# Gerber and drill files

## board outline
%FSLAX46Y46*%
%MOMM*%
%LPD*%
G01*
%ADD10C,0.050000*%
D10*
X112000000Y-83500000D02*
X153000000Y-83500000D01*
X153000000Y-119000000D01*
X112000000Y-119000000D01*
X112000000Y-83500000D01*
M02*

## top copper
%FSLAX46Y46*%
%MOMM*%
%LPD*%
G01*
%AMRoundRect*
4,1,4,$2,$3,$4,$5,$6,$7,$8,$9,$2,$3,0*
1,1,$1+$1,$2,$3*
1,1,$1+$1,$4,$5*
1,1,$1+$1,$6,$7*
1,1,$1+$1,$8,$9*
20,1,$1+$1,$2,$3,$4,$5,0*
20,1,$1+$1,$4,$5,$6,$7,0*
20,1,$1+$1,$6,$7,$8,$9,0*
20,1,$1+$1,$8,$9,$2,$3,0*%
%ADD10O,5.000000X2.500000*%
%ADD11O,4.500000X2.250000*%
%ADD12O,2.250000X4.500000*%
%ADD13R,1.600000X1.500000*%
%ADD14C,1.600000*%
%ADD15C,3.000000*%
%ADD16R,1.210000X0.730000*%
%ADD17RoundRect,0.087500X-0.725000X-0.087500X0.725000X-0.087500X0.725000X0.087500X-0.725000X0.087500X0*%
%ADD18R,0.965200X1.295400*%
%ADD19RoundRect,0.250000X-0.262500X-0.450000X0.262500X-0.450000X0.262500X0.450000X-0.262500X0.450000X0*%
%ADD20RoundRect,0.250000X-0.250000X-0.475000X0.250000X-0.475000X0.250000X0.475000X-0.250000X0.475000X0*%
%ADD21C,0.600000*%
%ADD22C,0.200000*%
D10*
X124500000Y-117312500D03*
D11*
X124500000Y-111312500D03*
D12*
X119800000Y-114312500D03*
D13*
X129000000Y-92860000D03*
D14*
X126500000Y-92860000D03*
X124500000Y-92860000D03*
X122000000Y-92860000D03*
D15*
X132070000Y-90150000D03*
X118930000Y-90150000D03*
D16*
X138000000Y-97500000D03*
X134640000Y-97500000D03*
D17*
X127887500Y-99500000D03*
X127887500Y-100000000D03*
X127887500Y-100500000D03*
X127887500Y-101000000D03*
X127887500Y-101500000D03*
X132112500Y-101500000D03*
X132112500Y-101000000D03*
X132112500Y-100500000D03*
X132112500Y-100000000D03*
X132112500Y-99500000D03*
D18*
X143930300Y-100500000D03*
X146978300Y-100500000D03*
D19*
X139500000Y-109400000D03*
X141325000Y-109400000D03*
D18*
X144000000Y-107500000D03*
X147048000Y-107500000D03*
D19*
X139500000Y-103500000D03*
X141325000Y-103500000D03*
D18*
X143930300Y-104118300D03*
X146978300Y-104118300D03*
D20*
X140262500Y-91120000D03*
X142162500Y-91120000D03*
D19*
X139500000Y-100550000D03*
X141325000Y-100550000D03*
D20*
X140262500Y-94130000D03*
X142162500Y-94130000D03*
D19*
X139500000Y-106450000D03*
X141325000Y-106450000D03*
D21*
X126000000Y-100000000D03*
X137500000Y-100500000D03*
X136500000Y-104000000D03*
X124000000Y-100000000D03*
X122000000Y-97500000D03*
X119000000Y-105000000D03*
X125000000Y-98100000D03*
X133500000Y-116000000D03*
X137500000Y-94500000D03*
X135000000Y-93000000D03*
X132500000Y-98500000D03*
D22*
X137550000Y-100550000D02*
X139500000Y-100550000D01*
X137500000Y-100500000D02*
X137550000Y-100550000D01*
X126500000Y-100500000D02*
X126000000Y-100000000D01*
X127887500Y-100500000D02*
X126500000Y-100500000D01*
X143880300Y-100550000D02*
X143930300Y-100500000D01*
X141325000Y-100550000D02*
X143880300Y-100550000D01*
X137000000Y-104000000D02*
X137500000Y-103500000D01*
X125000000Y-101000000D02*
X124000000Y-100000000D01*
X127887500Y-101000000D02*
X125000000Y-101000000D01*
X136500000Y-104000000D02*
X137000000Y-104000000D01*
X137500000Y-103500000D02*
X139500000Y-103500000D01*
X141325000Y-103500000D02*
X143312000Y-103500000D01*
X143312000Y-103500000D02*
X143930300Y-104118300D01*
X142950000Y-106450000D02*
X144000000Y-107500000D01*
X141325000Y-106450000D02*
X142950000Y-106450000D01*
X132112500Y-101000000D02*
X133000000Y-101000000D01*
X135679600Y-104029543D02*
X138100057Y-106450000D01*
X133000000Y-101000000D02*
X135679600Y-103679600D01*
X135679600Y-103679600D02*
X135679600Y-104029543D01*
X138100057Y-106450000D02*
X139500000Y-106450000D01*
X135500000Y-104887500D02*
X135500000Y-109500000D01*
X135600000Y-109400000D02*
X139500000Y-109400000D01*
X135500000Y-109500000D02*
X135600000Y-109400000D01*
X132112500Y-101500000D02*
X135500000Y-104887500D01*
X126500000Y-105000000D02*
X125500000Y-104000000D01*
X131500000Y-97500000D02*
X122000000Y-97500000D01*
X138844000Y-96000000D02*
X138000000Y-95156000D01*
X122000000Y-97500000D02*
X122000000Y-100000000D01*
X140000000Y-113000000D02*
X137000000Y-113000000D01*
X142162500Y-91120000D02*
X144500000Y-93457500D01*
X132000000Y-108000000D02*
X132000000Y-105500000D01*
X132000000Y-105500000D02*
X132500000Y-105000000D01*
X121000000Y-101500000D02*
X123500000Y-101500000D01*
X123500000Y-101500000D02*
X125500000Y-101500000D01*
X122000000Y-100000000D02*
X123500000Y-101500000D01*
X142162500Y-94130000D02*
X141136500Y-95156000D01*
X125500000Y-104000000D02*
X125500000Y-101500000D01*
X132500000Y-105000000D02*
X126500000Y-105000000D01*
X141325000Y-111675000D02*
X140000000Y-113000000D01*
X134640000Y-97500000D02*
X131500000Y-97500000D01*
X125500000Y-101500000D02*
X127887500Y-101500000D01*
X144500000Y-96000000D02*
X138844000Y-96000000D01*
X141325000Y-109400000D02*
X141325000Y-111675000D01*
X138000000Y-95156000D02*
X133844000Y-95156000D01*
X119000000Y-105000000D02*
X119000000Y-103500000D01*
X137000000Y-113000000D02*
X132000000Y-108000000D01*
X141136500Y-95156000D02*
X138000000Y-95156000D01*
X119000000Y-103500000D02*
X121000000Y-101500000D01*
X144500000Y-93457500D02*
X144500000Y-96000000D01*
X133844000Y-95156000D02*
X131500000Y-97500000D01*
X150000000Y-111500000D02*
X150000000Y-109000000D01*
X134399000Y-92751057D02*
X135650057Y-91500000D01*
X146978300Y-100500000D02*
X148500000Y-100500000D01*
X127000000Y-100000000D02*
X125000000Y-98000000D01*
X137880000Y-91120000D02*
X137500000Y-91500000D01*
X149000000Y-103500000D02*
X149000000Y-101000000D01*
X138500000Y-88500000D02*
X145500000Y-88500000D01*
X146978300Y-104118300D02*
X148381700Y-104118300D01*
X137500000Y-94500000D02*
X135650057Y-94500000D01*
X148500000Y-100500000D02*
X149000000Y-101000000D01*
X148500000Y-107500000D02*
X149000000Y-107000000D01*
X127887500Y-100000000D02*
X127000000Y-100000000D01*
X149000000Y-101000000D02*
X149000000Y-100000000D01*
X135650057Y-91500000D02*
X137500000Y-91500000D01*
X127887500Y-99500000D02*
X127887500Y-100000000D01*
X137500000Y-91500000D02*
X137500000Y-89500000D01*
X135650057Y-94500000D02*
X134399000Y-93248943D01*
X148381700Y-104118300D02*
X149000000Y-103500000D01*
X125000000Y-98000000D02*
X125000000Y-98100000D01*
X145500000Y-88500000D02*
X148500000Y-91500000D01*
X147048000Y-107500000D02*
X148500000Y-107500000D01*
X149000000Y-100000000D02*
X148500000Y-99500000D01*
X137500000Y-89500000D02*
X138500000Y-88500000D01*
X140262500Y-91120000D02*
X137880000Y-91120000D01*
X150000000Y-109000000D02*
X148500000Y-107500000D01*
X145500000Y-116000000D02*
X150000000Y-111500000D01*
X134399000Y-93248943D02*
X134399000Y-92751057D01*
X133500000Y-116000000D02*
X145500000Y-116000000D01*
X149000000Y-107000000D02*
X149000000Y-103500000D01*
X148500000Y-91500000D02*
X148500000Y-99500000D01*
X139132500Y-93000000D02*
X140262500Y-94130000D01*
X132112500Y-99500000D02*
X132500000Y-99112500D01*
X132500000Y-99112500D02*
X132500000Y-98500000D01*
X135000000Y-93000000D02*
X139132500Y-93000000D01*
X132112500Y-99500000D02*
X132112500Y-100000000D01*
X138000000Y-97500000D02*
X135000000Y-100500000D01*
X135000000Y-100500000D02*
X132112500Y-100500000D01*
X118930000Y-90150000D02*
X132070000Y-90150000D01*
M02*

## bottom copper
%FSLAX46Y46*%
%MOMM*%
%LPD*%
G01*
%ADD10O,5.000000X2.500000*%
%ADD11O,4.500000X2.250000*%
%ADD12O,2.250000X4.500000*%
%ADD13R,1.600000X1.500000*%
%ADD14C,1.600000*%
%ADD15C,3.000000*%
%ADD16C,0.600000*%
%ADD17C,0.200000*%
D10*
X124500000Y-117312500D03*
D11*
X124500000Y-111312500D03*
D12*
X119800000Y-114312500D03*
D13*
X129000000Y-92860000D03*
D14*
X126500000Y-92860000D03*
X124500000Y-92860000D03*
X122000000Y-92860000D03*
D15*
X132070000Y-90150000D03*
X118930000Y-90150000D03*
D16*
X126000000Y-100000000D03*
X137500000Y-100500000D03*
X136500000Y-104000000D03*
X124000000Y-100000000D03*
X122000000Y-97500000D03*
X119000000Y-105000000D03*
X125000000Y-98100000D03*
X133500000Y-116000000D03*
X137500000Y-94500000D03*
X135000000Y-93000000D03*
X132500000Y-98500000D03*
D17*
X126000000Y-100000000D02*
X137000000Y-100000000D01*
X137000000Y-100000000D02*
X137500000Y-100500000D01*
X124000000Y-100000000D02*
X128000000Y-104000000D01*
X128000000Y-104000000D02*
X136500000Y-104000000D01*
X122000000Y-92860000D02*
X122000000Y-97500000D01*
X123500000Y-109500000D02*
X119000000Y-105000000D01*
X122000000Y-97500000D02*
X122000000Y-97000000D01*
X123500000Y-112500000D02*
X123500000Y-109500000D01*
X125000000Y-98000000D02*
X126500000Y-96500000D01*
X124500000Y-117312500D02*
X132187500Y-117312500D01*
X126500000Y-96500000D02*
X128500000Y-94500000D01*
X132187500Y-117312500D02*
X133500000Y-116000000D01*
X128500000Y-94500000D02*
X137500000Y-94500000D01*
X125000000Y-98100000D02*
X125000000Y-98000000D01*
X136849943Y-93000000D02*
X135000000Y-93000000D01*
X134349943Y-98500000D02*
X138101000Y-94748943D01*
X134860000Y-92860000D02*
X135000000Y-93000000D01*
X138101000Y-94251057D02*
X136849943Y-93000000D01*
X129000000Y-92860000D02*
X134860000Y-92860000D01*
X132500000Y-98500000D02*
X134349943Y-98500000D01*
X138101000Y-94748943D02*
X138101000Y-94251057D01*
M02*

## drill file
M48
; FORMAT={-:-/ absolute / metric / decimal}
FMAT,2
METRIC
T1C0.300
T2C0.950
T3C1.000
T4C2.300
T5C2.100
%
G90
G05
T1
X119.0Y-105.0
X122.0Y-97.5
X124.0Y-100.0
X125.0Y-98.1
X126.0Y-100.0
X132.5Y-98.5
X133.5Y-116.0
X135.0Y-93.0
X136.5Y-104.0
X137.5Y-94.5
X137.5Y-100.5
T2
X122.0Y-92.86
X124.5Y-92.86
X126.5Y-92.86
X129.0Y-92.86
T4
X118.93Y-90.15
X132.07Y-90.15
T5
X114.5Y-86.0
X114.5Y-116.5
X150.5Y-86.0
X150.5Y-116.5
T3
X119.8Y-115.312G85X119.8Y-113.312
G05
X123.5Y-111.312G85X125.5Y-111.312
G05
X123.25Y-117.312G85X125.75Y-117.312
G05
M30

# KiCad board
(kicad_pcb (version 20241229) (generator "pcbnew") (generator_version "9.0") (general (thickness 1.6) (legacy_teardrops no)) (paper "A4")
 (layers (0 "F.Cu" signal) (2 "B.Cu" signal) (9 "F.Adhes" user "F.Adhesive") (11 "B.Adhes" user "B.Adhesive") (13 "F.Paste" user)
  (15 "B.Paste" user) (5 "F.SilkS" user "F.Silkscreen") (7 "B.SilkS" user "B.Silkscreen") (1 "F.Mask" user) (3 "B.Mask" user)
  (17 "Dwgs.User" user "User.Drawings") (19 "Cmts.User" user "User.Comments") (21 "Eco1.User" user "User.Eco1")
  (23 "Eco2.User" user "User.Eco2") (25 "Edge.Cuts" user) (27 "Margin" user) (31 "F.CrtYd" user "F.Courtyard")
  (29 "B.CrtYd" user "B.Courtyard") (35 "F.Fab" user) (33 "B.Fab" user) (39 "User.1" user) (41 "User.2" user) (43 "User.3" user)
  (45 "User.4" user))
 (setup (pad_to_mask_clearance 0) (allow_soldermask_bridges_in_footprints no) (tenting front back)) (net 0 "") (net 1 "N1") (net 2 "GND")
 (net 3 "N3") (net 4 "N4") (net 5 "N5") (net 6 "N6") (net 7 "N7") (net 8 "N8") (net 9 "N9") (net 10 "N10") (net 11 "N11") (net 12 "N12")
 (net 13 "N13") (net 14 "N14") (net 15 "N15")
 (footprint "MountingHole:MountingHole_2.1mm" (layer "F.Cu") (at 150.5 86)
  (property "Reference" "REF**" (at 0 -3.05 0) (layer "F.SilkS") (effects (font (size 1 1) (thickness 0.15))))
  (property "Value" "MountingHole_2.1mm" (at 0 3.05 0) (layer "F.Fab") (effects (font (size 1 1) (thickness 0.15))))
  (pad "" np_thru_hole circle (at 0 0) (size 2.1 2.1) (drill 2.1) (layers "*.Cu" "*.Mask")))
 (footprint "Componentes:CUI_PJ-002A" (layer "F.Cu") (at 124.5 117.3125 90)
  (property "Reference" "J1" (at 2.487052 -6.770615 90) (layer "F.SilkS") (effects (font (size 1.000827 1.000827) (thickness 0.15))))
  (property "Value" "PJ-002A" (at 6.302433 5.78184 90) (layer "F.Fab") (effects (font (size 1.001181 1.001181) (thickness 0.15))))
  (pad "1" thru_hole oval (at 0 0 90) (size 2.5 5) (drill oval 1 3.5) (layers "*.Cu" "*.Mask") (remove_unused_layers no) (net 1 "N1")
   (solder_mask_margin 0.102))
  (pad "2" thru_hole oval (at 6 0 90) (size 2.25 4.5) (drill oval 1 3) (layers "*.Cu" "*.Mask") (remove_unused_layers no) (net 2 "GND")
   (solder_mask_margin 0.102))
  (pad "3" thru_hole oval (at 3 -4.7 90) (size 4.5 2.25) (drill oval 3 1) (layers "*.Cu" "*.Mask") (remove_unused_layers no) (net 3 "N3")
   (solder_mask_margin 0.102)))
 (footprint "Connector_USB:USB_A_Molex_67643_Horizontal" (layer "F.Cu") (at 129 92.86 180)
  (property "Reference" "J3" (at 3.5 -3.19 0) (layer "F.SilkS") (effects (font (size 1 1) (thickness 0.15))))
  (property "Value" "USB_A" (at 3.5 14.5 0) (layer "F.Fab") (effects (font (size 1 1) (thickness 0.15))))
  (pad "1" thru_hole rect (at 0 0 180) (size 1.6 1.5) (drill 0.95) (layers "*.Cu" "*.Mask") (remove_unused_layers no) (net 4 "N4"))
  (pad "2" thru_hole circle (at 2.5 0 180) (size 1.6 1.6) (drill 0.95) (layers "*.Cu" "*.Mask") (remove_unused_layers no) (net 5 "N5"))
  (pad "3" thru_hole circle (at 4.5 0 180) (size 1.6 1.6) (drill 0.95) (layers "*.Cu" "*.Mask") (remove_unused_layers no) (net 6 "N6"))
  (pad "4" thru_hole circle (at 7 0 180) (size 1.6 1.6) (drill 0.95) (layers "*.Cu" "*.Mask") (remove_unused_layers no) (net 2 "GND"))
  (pad "5" thru_hole circle (at -3.07 2.71 180) (size 3 3) (drill 2.3) (layers "*.Cu" "*.Mask") (remove_unused_layers no) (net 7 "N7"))
  (pad "5" thru_hole circle (at 10.07 2.71 180) (size 3 3) (drill 2.3) (layers "*.Cu" "*.Mask") (remove_unused_layers no) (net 7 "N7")))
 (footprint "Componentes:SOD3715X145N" (layer "F.Cu") (at 136.32 97.5)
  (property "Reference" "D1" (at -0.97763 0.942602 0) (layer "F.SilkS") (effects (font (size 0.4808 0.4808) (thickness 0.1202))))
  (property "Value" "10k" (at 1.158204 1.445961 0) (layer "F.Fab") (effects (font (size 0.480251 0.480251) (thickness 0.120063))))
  (pad "A" smd rect (at 1.68 0) (size 1.21 0.73) (layers "F.Cu" "F.Mask" "F.Paste") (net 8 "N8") (solder_mask_margin 0.102))
  (pad "C" smd rect (at -1.68 0) (size 1.21 0.73) (layers "F.Cu" "F.Mask" "F.Paste") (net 2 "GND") (solder_mask_margin 0.102)))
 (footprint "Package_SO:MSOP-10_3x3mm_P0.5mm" (layer "F.Cu") (at 130 100.5)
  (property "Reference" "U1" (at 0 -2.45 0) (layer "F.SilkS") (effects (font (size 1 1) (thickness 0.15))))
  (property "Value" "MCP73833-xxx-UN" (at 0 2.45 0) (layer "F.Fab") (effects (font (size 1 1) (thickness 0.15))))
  (pad "1" smd roundrect (at -2.1125 -1) (size 1.625 0.35) (layers "F.Cu" "F.Mask" "F.Paste") (roundrect_rratio 0.25) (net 1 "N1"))
  (pad "2" smd roundrect (at -2.1125 -0.5) (size 1.625 0.35) (layers "F.Cu" "F.Mask" "F.Paste") (roundrect_rratio 0.25) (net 1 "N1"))
  (pad "3" smd roundrect (at -2.1125 0) (size 1.625 0.35) (layers "F.Cu" "F.Mask" "F.Paste") (roundrect_rratio 0.25) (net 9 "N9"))
  (pad "4" smd roundrect (at -2.1125 0.5) (size 1.625 0.35) (layers "F.Cu" "F.Mask" "F.Paste") (roundrect_rratio 0.25) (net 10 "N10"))
  (pad "5" smd roundrect (at -2.1125 1) (size 1.625 0.35) (layers "F.Cu" "F.Mask" "F.Paste") (roundrect_rratio 0.25) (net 2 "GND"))
  (pad "6" smd roundrect (at 2.1125 1) (size 1.625 0.35) (layers "F.Cu" "F.Mask" "F.Paste") (roundrect_rratio 0.25) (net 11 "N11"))
  (pad "7" smd roundrect (at 2.1125 0.5) (size 1.625 0.35) (layers "F.Cu" "F.Mask" "F.Paste") (roundrect_rratio 0.25) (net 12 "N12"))
  (pad "8" smd roundrect (at 2.1125 0) (size 1.625 0.35) (layers "F.Cu" "F.Mask" "F.Paste") (roundrect_rratio 0.25) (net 8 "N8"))
  (pad "9" smd roundrect (at 2.1125 -0.5) (size 1.625 0.35) (layers "F.Cu" "F.Mask" "F.Paste") (roundrect_rratio 0.25) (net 4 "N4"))
  (pad "10" smd roundrect (at 2.1125 -1) (size 1.625 0.35) (layers "F.Cu" "F.Mask" "F.Paste") (roundrect_rratio 0.25) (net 4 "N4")))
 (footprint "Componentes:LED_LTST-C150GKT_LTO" (layer "F.Cu") (at 145.4543 100.5)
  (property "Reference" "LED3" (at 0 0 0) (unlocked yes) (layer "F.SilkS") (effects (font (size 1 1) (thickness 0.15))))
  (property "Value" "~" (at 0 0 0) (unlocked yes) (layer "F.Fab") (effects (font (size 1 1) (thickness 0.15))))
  (pad "1" smd rect (at -1.524 0) (size 0.9652 1.2954) (layers "F.Cu" "F.Mask" "F.Paste") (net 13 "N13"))
  (pad "2" smd rect (at 1.524 0) (size 0.9652 1.2954) (layers "F.Cu" "F.Mask" "F.Paste") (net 1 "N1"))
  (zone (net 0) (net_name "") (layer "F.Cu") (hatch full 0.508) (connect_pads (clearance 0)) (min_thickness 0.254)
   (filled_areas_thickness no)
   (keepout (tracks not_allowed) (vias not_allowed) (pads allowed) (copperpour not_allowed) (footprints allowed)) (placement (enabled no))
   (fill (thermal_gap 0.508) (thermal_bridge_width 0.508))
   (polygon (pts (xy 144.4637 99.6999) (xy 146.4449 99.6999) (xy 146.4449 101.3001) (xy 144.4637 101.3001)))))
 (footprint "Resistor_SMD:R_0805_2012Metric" (layer "F.Cu") (at 140.4125 109.4)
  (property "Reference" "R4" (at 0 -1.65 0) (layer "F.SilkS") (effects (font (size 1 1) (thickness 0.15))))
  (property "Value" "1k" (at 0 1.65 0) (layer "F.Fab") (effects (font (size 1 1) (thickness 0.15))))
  (pad "1" smd roundrect (at -0.9125 0) (size 1.025 1.4) (layers "F.Cu" "F.Mask" "F.Paste") (roundrect_rratio 0.243902) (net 11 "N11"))
  (pad "2" smd roundrect (at 0.9125 0) (size 1.025 1.4) (layers "F.Cu" "F.Mask" "F.Paste") (roundrect_rratio 0.243902) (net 2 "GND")))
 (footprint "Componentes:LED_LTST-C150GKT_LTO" (layer "F.Cu") (at 145.524 107.5)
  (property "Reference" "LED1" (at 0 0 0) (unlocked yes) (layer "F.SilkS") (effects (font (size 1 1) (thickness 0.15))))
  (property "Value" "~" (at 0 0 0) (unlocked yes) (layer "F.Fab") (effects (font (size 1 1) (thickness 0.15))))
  (pad "1" smd rect (at -1.524 0) (size 0.9652 1.2954) (layers "F.Cu" "F.Mask" "F.Paste") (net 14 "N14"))
  (pad "2" smd rect (at 1.524 0) (size 0.9652 1.2954) (layers "F.Cu" "F.Mask" "F.Paste") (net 1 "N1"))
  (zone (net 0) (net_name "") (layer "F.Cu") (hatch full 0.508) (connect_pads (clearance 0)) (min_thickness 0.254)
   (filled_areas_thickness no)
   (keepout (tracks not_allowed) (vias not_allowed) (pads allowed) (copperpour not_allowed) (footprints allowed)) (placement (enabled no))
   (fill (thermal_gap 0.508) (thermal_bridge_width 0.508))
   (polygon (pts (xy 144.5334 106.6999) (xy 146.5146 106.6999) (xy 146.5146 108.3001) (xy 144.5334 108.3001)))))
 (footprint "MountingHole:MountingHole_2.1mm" (layer "F.Cu") (at 114.5 86)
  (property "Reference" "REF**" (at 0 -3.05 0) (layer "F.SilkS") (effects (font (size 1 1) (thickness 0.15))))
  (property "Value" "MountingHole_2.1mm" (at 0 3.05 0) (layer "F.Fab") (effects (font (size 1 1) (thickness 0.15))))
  (pad "" np_thru_hole circle (at 0 0) (size 2.1 2.1) (drill 2.1) (layers "*.Cu" "*.Mask")))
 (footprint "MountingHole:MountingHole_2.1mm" (layer "F.Cu") (at 114.5 116.5)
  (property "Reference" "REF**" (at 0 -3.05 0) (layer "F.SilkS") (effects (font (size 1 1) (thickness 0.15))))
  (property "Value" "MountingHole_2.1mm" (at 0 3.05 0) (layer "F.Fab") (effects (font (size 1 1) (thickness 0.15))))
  (pad "" np_thru_hole circle (at 0 0) (size 2.1 2.1) (drill 2.1) (layers "*.Cu" "*.Mask")))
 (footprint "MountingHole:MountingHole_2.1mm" (layer "F.Cu") (at 150.5 116.5)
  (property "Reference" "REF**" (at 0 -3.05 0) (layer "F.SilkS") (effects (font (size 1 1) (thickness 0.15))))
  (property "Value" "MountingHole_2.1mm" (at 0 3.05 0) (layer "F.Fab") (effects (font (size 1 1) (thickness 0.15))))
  (pad "" np_thru_hole circle (at 0 0) (size 2.1 2.1) (drill 2.1) (layers "*.Cu" "*.Mask")))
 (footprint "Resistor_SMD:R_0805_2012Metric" (layer "F.Cu") (at 140.4125 103.5)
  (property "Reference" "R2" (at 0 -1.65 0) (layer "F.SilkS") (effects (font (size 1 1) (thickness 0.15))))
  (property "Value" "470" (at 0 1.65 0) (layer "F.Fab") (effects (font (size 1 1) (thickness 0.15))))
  (pad "1" smd roundrect (at -0.9125 0) (size 1.025 1.4) (layers "F.Cu" "F.Mask" "F.Paste") (roundrect_rratio 0.243902) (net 10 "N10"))
  (pad "2" smd roundrect (at 0.9125 0) (size 1.025 1.4) (layers "F.Cu" "F.Mask" "F.Paste") (roundrect_rratio 0.243902) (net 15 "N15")))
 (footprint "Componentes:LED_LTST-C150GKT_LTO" (layer "F.Cu") (at 145.4543 104.1183)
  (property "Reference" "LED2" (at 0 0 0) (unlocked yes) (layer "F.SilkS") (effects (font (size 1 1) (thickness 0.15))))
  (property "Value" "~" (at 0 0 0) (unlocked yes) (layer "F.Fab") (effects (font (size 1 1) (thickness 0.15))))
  (pad "1" smd rect (at -1.524 0) (size 0.9652 1.2954) (layers "F.Cu" "F.Mask" "F.Paste") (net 15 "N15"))
  (pad "2" smd rect (at 1.524 0) (size 0.9652 1.2954) (layers "F.Cu" "F.Mask" "F.Paste") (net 1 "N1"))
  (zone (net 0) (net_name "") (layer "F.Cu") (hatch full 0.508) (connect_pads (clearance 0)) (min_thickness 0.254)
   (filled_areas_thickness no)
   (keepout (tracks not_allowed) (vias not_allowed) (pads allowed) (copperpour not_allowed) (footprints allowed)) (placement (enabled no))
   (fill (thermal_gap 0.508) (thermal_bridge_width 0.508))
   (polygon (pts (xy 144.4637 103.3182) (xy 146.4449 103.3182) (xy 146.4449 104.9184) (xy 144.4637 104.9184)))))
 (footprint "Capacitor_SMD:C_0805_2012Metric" (layer "F.Cu") (at 141.2125 91.12)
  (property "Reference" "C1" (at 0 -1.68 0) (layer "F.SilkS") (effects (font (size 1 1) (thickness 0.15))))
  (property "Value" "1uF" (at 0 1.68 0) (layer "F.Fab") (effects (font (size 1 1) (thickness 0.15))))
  (pad "1" smd roundrect (at -0.95 0) (size 1 1.45) (layers "F.Cu" "F.Mask" "F.Paste") (roundrect_rratio 0.25) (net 1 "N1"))
  (pad "2" smd roundrect (at 0.95 0) (size 1 1.45) (layers "F.Cu" "F.Mask" "F.Paste") (roundrect_rratio 0.25) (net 2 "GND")))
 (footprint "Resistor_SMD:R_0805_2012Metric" (layer "F.Cu") (at 140.4125 100.55)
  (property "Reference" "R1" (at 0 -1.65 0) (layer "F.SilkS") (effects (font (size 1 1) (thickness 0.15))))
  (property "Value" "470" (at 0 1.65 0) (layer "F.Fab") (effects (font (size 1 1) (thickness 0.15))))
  (pad "1" smd roundrect (at -0.9125 0) (size 1.025 1.4) (layers "F.Cu" "F.Mask" "F.Paste") (roundrect_rratio 0.243902) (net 9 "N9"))
  (pad "2" smd roundrect (at 0.9125 0) (size 1.025 1.4) (layers "F.Cu" "F.Mask" "F.Paste") (roundrect_rratio 0.243902) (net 13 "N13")))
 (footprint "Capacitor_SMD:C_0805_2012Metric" (layer "F.Cu") (at 141.2125 94.13)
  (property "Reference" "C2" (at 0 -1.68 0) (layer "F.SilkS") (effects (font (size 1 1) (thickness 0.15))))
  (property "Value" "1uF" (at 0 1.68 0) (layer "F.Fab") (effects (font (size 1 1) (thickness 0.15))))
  (pad "1" smd roundrect (at -0.95 0) (size 1 1.45) (layers "F.Cu" "F.Mask" "F.Paste") (roundrect_rratio 0.25) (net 4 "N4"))
  (pad "2" smd roundrect (at 0.95 0) (size 1 1.45) (layers "F.Cu" "F.Mask" "F.Paste") (roundrect_rratio 0.25) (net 2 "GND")))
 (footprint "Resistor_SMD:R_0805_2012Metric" (layer "F.Cu") (at 140.4125 106.45)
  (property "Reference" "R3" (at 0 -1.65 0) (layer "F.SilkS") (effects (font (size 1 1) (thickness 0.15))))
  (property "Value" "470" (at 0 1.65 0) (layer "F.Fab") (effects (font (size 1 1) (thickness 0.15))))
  (pad "1" smd roundrect (at -0.9125 0) (size 1.025 1.4) (layers "F.Cu" "F.Mask" "F.Paste") (roundrect_rratio 0.243902) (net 12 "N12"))
  (pad "2" smd roundrect (at 0.9125 0) (size 1.025 1.4) (layers "F.Cu" "F.Mask" "F.Paste") (roundrect_rratio 0.243902) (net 14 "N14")))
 (gr_rect (start 112 83.5) (end 153 119) (stroke (width 0.05) (type default)) (fill no) (layer "Edge.Cuts"))
 (segment (start 137.55 100.55) (end 139.5 100.55) (width 0.2) (layer "F.Cu") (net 9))
 (segment (start 137.5 100.5) (end 137.55 100.55) (width 0.2) (layer "F.Cu") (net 9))
 (segment (start 126.5 100.5) (end 126 100) (width 0.2) (layer "F.Cu") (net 9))
 (segment (start 127.8875 100.5) (end 126.5 100.5) (width 0.2) (layer "F.Cu") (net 9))
 (via (at 126 100) (size 0.6) (drill 0.3) (layers "F.Cu" "B.Cu") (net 9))
 (via (at 137.5 100.5) (size 0.6) (drill 0.3) (layers "F.Cu" "B.Cu") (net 9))
 (segment (start 126 100) (end 137 100) (width 0.2) (layer "B.Cu") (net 9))
 (segment (start 137 100) (end 137.5 100.5) (width 0.2) (layer "B.Cu") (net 9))
 (segment (start 143.8803 100.55) (end 143.9303 100.5) (width 0.2) (layer "F.Cu") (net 13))
 (segment (start 141.325 100.55) (end 143.8803 100.55) (width 0.2) (layer "F.Cu") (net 13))
 (segment (start 137 104) (end 137.5 103.5) (width 0.2) (layer "F.Cu") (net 10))
 (segment (start 125 101) (end 124 100) (width 0.2) (layer "F.Cu") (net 10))
 (segment (start 127.8875 101) (end 125 101) (width 0.2) (layer "F.Cu") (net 10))
 (segment (start 136.5 104) (end 137 104) (width 0.2) (layer "F.Cu") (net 10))
 (segment (start 137.5 103.5) (end 139.5 103.5) (width 0.2) (layer "F.Cu") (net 10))
 (via (at 136.5 104) (size 0.6) (drill 0.3) (layers "F.Cu" "B.Cu") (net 10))
 (via (at 124 100) (size 0.6) (drill 0.3) (layers "F.Cu" "B.Cu") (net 10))
 (segment (start 124 100) (end 128 104) (width 0.2) (layer "B.Cu") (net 10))
 (segment (start 128 104) (end 136.5 104) (width 0.2) (layer "B.Cu") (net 10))
 (segment (start 141.325 103.5) (end 143.312 103.5) (width 0.2) (layer "F.Cu") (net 15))
 (segment (start 143.312 103.5) (end 143.9303 104.1183) (width 0.2) (layer "F.Cu") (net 15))
 (segment (start 142.95 106.45) (end 144 107.5) (width 0.2) (layer "F.Cu") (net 14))
 (segment (start 141.325 106.45) (end 142.95 106.45) (width 0.2) (layer "F.Cu") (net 14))
 (segment (start 132.1125 101) (end 133 101) (width 0.2) (layer "F.Cu") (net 12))
 (segment (start 135.6796 104.029543) (end 138.100057 106.45) (width 0.2) (layer "F.Cu") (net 12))
 (segment (start 133 101) (end 135.6796 103.6796) (width 0.2) (layer "F.Cu") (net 12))
 (segment (start 135.6796 103.6796) (end 135.6796 104.029543) (width 0.2) (layer "F.Cu") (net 12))
 (segment (start 138.100057 106.45) (end 139.5 106.45) (width 0.2) (layer "F.Cu") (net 12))
 (segment (start 135.5 104.8875) (end 135.5 109.5) (width 0.2) (layer "F.Cu") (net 11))
 (segment (start 135.6 109.4) (end 139.5 109.4) (width 0.2) (layer "F.Cu") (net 11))
 (segment (start 135.5 109.5) (end 135.6 109.4) (width 0.2) (layer "F.Cu") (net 11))
 (segment (start 132.1125 101.5) (end 135.5 104.8875) (width 0.2) (layer "F.Cu") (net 11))
 (segment (start 126.5 105) (end 125.5 104) (width 0.2) (layer "F.Cu") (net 2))
 (segment (start 131.5 97.5) (end 122 97.5) (width 0.2) (layer "F.Cu") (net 2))
 (segment (start 138.844 96) (end 138 95.156) (width 0.2) (layer "F.Cu") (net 2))
 (segment (start 122 97.5) (end 122 100) (width 0.2) (layer "F.Cu") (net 2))
 (segment (start 140 113) (end 137 113) (width 0.2) (layer "F.Cu") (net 2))
 (segment (start 142.1625 91.12) (end 144.5 93.4575) (width 0.2) (layer "F.Cu") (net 2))
 (segment (start 132 108) (end 132 105.5) (width 0.2) (layer "F.Cu") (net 2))
 (segment (start 132 105.5) (end 132.5 105) (width 0.2) (layer "F.Cu") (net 2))
 (segment (start 121 101.5) (end 123.5 101.5) (width 0.2) (layer "F.Cu") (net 2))
 (segment (start 123.5 101.5) (end 125.5 101.5) (width 0.2) (layer "F.Cu") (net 2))
 (segment (start 122 100) (end 123.5 101.5) (width 0.2) (layer "F.Cu") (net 2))
 (segment (start 142.1625 94.13) (end 141.1365 95.156) (width 0.2) (layer "F.Cu") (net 2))
 (segment (start 125.5 104) (end 125.5 101.5) (width 0.2) (layer "F.Cu") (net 2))
 (segment (start 132.5 105) (end 126.5 105) (width 0.2) (layer "F.Cu") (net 2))
 (segment (start 141.325 111.675) (end 140 113) (width 0.2) (layer "F.Cu") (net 2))
 (segment (start 134.64 97.5) (end 131.5 97.5) (width 0.2) (layer "F.Cu") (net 2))
 (segment (start 125.5 101.5) (end 127.8875 101.5) (width 0.2) (layer "F.Cu") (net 2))
 (segment (start 144.5 96) (end 138.844 96) (width 0.2) (layer "F.Cu") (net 2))
 (segment (start 141.325 109.4) (end 141.325 111.675) (width 0.2) (layer "F.Cu") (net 2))
 (segment (start 138 95.156) (end 133.844 95.156) (width 0.2) (layer "F.Cu") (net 2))
 (segment (start 119 105) (end 119 103.5) (width 0.2) (layer "F.Cu") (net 2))
 (segment (start 137 113) (end 132 108) (width 0.2) (layer "F.Cu") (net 2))
 (segment (start 141.1365 95.156) (end 138 95.156) (width 0.2) (layer "F.Cu") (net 2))
 (segment (start 119 103.5) (end 121 101.5) (width 0.2) (layer "F.Cu") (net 2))
 (segment (start 144.5 93.4575) (end 144.5 96) (width 0.2) (layer "F.Cu") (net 2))
 (segment (start 133.844 95.156) (end 131.5 97.5) (width 0.2) (layer "F.Cu") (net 2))
 (via (at 122 97.5) (size 0.6) (drill 0.3) (layers "F.Cu" "B.Cu") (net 2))
 (via (at 119 105) (size 0.6) (drill 0.3) (layers "F.Cu" "B.Cu") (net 2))
 (segment (start 122 92.86) (end 122 97.5) (width 0.2) (layer "B.Cu") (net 2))
 (segment (start 123.5 109.5) (end 119 105) (width 0.2) (layer "B.Cu") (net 2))
 (segment (start 122 97.5) (end 122 97) (width 0.2) (layer "B.Cu") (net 2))
 (segment (start 123.5 112.5) (end 123.5 109.5) (width 0.2) (layer "B.Cu") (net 2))
 (segment (start 150 111.5) (end 150 109) (width 0.2) (layer "F.Cu") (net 1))
 (segment (start 134.399 92.751057) (end 135.650057 91.5) (width 0.2) (layer "F.Cu") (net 1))
 (segment (start 146.9783 100.5) (end 148.5 100.5) (width 0.2) (layer "F.Cu") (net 1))
 (segment (start 127 100) (end 125 98) (width 0.2) (layer "F.Cu") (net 1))
 (segment (start 137.88 91.12) (end 137.5 91.5) (width 0.2) (layer "F.Cu") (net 1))
 (segment (start 149 103.5) (end 149 101) (width 0.2) (layer "F.Cu") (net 1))
 (segment (start 138.5 88.5) (end 145.5 88.5) (width 0.2) (layer "F.Cu") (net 1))
 (segment (start 146.9783 104.1183) (end 148.3817 104.1183) (width 0.2) (layer "F.Cu") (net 1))
 (segment (start 137.5 94.5) (end 135.650057 94.5) (width 0.2) (layer "F.Cu") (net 1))
 (segment (start 148.5 100.5) (end 149 101) (width 0.2) (layer "F.Cu") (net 1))
 (segment (start 148.5 107.5) (end 149 107) (width 0.2) (layer "F.Cu") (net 1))
 (segment (start 127.8875 100) (end 127 100) (width 0.2) (layer "F.Cu") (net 1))
 (segment (start 149 101) (end 149 100) (width 0.2) (layer "F.Cu") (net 1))
 (segment (start 135.650057 91.5) (end 137.5 91.5) (width 0.2) (layer "F.Cu") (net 1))
 (segment (start 127.8875 99.5) (end 127.8875 100) (width 0.2) (layer "F.Cu") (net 1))
 (segment (start 137.5 91.5) (end 137.5 89.5) (width 0.2) (layer "F.Cu") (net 1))
 (segment (start 135.650057 94.5) (end 134.399 93.248943) (width 0.2) (layer "F.Cu") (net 1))
 (segment (start 148.3817 104.1183) (end 149 103.5) (width 0.2) (layer "F.Cu") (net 1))
 (segment (start 125 98) (end 125 98.1) (width 0.2) (layer "F.Cu") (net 1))
 (segment (start 145.5 88.5) (end 148.5 91.5) (width 0.2) (layer "F.Cu") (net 1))
 (segment (start 147.048 107.5) (end 148.5 107.5) (width 0.2) (layer "F.Cu") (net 1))
 (segment (start 149 100) (end 148.5 99.5) (width 0.2) (layer "F.Cu") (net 1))
 (segment (start 137.5 89.5) (end 138.5 88.5) (width 0.2) (layer "F.Cu") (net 1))
 (segment (start 140.2625 91.12) (end 137.88 91.12) (width 0.2) (layer "F.Cu") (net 1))
 (segment (start 150 109) (end 148.5 107.5) (width 0.2) (layer "F.Cu") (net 1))
 (segment (start 145.5 116) (end 150 111.5) (width 0.2) (layer "F.Cu") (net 1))
 (segment (start 134.399 93.248943) (end 134.399 92.751057) (width 0.2) (layer "F.Cu") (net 1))
 (segment (start 133.5 116) (end 145.5 116) (width 0.2) (layer "F.Cu") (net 1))
 (segment (start 149 107) (end 149 103.5) (width 0.2) (layer "F.Cu") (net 1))
 (segment (start 148.5 91.5) (end 148.5 99.5) (width 0.2) (layer "F.Cu") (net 1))
 (via (at 125 98.1) (size 0.6) (drill 0.3) (layers "F.Cu" "B.Cu") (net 1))
 (via (at 133.5 116) (size 0.6) (drill 0.3) (layers "F.Cu" "B.Cu") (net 1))
 (via (at 137.5 94.5) (size 0.6) (drill 0.3) (layers "F.Cu" "B.Cu") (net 1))
 (segment (start 125 98) (end 126.5 96.5) (width 0.2) (layer "B.Cu") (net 1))
 (segment (start 124.5 117.3125) (end 132.1875 117.3125) (width 0.2) (layer "B.Cu") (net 1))
 (segment (start 126.5 96.5) (end 128.5 94.5) (width 0.2) (layer "B.Cu") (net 1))
 (segment (start 132.1875 117.3125) (end 133.5 116) (width 0.2) (layer "B.Cu") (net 1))
 (segment (start 128.5 94.5) (end 137.5 94.5) (width 0.2) (layer "B.Cu") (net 1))
 (segment (start 125 98.1) (end 125 98) (width 0.2) (layer "B.Cu") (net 1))
 (segment (start 139.1325 93) (end 140.2625 94.13) (width 0.2) (layer "F.Cu") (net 4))
 (segment (start 132.1125 99.5) (end 132.5 99.1125) (width 0.2) (layer "F.Cu") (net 4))
 (segment (start 132.5 99.1125) (end 132.5 98.5) (width 0.2) (layer "F.Cu") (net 4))
 (segment (start 135 93) (end 139.1325 93) (width 0.2) (layer "F.Cu") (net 4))
 (segment (start 132.1125 99.5) (end 132.1125 100) (width 0.2) (layer "F.Cu") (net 4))
 (via (at 135 93) (size 0.6) (drill 0.3) (layers "F.Cu" "B.Cu") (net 4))
 (via (at 132.5 98.5) (size 0.6) (drill 0.3) (layers "F.Cu" "B.Cu") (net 4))
 (segment (start 136.849943 93) (end 135 93) (width 0.2) (layer "B.Cu") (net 4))
 (segment (start 134.349943 98.5) (end 138.101 94.748943) (width 0.2) (layer "B.Cu") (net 4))
 (segment (start 134.86 92.86) (end 135 93) (width 0.2) (layer "B.Cu") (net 4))
 (segment (start 138.101 94.251057) (end 136.849943 93) (width 0.2) (layer "B.Cu") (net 4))
 (segment (start 129 92.86) (end 134.86 92.86) (width 0.2) (layer "B.Cu") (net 4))
 (segment (start 132.5 98.5) (end 134.349943 98.5) (width 0.2) (layer "B.Cu") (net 4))
 (segment (start 138.101 94.748943) (end 138.101 94.251057) (width 0.2) (layer "B.Cu") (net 4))
 (segment (start 138 97.5) (end 135 100.5) (width 0.2) (layer "F.Cu") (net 8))
 (segment (start 135 100.5) (end 132.1125 100.5) (width 0.2) (layer "F.Cu") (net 8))
 (segment (start 118.93 90.15) (end 132.07 90.15) (width 0.2) (layer "F.Cu") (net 7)))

